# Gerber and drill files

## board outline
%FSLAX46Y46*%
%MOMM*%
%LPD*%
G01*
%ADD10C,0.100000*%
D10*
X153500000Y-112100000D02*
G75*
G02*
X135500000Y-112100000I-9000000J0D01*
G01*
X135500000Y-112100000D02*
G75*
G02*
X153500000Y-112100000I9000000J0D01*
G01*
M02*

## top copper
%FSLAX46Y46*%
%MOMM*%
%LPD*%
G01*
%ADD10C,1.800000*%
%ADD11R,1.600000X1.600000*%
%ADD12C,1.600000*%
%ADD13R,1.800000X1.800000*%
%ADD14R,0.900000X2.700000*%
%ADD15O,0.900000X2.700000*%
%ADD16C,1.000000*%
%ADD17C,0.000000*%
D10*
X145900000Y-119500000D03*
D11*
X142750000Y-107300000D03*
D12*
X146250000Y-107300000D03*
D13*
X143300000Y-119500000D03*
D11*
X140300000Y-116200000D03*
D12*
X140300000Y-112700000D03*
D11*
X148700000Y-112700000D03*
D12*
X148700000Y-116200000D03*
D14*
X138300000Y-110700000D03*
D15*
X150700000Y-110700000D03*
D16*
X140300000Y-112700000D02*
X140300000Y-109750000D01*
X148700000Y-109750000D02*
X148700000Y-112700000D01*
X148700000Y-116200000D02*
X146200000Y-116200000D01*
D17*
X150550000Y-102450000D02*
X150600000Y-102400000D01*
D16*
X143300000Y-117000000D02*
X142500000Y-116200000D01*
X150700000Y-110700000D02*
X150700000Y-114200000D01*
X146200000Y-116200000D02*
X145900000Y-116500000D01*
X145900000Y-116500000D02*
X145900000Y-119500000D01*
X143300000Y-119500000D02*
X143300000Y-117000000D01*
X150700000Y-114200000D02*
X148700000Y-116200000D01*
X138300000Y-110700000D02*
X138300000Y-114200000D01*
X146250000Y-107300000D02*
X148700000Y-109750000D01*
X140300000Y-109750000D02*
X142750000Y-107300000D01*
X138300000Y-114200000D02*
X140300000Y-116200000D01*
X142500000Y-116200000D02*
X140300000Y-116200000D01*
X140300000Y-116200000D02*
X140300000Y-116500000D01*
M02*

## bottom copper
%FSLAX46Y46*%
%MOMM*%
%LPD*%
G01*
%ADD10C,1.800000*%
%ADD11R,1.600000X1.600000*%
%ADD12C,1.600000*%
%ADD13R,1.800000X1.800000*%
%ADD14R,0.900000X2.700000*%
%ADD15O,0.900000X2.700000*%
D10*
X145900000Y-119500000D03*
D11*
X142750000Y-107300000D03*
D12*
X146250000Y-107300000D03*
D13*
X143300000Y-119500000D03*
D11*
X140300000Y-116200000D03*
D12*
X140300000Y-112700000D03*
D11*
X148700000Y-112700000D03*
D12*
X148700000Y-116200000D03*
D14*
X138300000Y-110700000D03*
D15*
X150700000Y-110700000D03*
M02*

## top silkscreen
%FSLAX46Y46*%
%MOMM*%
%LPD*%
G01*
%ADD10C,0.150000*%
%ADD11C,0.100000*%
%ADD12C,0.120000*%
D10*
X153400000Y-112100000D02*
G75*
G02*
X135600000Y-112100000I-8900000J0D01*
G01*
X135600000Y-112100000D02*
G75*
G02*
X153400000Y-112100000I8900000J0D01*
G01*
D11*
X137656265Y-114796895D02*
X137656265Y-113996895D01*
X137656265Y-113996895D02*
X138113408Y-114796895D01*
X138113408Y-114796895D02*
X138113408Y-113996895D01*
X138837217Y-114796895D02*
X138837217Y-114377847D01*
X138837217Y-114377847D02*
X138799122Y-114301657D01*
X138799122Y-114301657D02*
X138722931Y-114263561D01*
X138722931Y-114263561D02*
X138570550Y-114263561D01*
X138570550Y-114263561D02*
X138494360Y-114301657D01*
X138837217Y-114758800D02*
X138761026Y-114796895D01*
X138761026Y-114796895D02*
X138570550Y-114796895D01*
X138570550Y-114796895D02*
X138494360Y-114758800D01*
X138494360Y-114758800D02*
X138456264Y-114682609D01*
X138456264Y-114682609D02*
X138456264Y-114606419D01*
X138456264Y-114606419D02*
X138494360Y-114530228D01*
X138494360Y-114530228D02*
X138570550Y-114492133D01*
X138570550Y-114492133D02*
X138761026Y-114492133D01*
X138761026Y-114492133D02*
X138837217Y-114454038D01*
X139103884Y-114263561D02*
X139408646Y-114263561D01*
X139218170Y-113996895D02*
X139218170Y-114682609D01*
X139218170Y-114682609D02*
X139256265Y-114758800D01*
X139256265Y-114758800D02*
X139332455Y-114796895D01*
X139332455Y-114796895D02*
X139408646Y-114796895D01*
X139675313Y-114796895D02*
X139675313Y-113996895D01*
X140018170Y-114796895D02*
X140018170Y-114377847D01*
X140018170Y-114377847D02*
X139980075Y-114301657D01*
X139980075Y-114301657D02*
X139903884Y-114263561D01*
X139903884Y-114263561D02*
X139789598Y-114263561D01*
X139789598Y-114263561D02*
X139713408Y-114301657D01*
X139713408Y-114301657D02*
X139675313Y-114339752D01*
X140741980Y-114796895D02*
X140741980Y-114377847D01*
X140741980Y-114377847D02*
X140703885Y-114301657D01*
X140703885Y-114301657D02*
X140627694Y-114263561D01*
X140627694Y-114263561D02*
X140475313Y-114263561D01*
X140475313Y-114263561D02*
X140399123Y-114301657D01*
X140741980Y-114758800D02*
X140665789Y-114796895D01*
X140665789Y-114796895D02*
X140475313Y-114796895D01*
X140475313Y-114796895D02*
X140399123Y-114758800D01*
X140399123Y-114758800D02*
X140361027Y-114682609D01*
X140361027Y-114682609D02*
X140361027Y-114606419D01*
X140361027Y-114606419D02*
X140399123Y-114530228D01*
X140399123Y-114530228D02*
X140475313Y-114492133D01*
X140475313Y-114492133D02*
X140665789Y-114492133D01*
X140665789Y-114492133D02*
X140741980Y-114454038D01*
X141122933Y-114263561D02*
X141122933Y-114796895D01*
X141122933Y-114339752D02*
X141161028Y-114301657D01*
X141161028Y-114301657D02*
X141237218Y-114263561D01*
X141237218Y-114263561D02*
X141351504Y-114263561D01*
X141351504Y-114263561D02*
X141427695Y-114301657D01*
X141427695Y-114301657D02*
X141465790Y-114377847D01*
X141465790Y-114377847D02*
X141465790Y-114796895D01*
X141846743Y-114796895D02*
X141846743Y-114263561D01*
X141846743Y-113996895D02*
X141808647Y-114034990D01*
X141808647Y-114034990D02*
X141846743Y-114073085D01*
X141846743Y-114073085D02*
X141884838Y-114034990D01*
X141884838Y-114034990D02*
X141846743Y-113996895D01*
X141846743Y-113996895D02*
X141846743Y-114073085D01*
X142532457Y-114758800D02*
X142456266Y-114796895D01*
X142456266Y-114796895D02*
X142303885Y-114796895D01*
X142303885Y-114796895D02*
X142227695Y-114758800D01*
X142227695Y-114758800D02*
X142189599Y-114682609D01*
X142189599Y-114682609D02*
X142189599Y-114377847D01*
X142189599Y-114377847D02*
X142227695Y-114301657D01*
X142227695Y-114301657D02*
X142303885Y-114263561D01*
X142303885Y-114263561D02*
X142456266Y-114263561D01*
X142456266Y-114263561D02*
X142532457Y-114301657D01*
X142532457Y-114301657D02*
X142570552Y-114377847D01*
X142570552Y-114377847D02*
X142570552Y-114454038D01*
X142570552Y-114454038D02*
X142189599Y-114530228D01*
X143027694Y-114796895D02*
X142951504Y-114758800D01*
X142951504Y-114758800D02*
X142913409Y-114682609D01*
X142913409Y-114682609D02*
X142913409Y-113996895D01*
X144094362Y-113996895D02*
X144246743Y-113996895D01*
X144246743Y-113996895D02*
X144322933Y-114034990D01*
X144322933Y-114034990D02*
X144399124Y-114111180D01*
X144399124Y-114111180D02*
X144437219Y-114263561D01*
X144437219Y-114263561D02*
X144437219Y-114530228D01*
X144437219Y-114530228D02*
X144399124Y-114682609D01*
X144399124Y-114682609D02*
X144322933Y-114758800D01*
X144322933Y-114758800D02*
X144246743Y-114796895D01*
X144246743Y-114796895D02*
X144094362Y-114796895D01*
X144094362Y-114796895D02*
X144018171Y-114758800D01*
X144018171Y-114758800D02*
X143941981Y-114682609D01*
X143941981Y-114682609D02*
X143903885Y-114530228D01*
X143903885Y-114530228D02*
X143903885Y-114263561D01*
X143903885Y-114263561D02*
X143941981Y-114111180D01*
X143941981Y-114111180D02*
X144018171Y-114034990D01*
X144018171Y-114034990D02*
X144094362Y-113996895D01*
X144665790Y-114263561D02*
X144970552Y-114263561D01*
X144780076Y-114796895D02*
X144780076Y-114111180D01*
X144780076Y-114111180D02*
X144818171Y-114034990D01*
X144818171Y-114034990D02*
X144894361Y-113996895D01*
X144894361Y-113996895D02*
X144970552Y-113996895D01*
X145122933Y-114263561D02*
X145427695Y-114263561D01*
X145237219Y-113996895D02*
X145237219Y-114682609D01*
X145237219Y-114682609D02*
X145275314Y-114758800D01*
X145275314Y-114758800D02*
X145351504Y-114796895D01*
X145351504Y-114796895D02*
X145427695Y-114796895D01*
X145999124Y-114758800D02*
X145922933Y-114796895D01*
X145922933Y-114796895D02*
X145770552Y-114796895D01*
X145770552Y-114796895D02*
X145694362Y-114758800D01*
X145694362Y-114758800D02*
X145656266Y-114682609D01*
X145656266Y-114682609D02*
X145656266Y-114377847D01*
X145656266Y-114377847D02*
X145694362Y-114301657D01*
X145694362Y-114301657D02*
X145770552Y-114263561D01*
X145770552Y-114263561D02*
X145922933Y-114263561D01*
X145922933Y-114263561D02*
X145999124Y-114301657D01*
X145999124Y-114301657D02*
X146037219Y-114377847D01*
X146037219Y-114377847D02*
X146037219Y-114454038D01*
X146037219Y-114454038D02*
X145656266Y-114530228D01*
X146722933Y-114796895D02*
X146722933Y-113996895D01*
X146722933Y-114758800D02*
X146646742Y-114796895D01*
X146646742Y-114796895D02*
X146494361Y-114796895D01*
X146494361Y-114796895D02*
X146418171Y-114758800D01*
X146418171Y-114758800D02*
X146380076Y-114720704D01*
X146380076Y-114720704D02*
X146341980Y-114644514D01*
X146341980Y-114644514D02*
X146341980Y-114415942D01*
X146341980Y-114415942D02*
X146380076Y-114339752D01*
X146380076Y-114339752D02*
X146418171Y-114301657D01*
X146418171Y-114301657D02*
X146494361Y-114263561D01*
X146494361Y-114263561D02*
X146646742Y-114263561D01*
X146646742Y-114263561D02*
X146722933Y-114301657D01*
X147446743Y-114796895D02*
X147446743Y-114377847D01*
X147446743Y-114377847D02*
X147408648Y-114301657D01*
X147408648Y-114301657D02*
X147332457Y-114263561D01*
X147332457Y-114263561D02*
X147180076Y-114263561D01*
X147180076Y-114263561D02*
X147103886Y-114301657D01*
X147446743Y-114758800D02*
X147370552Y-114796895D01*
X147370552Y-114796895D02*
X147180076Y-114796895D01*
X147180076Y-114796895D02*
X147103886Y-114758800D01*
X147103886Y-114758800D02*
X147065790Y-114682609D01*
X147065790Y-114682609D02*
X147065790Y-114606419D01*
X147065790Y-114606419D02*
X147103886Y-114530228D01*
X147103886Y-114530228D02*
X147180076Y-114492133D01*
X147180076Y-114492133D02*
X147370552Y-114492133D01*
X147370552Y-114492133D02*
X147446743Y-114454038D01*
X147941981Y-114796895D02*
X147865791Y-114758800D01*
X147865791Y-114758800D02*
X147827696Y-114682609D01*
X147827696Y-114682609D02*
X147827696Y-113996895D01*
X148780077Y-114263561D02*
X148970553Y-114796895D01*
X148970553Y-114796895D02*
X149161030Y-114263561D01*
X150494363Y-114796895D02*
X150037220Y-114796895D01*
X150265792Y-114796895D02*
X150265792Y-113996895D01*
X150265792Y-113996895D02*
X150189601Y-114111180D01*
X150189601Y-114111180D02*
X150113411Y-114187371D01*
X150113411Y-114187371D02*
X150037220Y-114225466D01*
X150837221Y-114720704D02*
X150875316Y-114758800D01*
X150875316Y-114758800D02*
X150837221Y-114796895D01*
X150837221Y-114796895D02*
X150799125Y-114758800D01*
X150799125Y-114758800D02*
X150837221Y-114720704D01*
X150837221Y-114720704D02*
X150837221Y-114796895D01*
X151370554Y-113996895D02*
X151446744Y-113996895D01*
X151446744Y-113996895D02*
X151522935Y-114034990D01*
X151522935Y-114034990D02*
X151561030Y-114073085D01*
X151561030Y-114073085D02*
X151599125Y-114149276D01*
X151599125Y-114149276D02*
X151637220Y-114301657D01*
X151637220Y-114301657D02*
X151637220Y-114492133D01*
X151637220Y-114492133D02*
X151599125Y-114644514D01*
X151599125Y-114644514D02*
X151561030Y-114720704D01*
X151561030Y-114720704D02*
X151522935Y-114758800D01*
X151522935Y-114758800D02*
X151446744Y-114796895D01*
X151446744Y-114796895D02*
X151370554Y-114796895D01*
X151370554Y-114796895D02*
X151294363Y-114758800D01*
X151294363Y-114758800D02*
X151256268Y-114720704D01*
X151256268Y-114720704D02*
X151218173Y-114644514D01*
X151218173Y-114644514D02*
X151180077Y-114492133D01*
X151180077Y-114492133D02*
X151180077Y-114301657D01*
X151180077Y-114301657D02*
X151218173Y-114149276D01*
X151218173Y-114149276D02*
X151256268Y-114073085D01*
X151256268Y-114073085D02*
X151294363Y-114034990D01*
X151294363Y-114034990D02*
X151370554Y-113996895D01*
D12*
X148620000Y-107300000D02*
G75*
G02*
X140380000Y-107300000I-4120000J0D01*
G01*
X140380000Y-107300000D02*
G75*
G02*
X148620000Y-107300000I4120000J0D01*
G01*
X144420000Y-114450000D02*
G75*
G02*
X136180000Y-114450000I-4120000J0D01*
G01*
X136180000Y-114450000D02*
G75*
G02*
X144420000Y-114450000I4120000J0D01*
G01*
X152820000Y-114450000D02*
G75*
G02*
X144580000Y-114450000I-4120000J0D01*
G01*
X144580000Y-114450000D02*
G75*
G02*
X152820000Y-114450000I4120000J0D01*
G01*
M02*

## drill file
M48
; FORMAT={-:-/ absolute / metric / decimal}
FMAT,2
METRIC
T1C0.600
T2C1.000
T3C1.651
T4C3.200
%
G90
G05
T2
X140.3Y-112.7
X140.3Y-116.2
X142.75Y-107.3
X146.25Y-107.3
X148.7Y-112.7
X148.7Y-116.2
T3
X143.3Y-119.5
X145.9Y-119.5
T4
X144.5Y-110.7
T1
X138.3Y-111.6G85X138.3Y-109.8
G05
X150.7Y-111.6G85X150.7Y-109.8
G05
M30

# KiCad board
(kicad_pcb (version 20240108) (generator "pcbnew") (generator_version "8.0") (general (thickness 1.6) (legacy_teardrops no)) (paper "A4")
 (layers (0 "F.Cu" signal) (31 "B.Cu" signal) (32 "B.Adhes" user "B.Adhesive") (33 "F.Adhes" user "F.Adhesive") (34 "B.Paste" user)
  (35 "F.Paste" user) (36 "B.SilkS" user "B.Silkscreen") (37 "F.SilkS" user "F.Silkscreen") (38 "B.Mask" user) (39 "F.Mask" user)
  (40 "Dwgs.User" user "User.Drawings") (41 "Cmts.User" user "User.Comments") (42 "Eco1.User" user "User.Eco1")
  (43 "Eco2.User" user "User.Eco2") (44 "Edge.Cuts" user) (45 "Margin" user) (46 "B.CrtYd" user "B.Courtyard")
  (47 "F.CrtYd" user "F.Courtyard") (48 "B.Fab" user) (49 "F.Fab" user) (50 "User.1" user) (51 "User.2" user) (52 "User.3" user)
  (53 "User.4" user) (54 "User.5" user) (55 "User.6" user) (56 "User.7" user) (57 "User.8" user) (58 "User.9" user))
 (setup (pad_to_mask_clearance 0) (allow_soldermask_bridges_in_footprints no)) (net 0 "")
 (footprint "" (layer "F.Cu") (at 145.9 119.5)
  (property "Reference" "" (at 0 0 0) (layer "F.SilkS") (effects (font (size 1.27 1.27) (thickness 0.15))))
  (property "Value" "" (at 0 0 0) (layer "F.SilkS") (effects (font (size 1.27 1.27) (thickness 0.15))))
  (pad "2" thru_hole circle (at 0 0) (size 1.8 1.8) (drill 1.651) (layers "*.Cu" "*.Mask") (remove_unused_layers no)))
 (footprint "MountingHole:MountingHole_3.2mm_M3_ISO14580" (layer "F.Cu") (at 144.5 110.7)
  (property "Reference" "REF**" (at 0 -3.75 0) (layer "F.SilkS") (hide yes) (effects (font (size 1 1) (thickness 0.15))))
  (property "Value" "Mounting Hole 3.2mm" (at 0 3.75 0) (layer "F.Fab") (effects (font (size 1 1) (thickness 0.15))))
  (pad "" np_thru_hole circle (at 0 0) (size 3.2 3.2) (drill 3.2) (layers "F&B.Cu" "*.Mask" "B.Paste")))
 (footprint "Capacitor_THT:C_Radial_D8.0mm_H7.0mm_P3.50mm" (layer "F.Cu") (at 142.75 107.3)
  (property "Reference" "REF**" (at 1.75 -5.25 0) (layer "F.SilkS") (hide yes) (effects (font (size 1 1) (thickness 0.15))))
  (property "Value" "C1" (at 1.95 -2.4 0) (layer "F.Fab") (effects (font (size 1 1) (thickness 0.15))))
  (fp_circle (center 1.75 0) (end 5.87 0) (stroke (width 0.12) (type solid)) (fill none) (layer "F.SilkS"))
  (pad "1" thru_hole rect (at 0 0) (size 1.6 1.6) (drill 1) (layers "*.Cu" "*.Mask") (remove_unused_layers no))
  (pad "2" thru_hole circle (at 3.5 0) (size 1.6 1.6) (drill 1) (layers "*.Cu" "*.Mask") (remove_unused_layers no)))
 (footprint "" (layer "F.Cu") (at 143.3 119.5)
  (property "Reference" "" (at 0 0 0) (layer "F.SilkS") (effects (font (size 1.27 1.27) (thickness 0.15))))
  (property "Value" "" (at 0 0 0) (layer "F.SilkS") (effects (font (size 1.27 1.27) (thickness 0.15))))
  (pad "1" thru_hole rect (at 0 0) (size 1.8 1.8) (drill 1.651) (layers "*.Cu" "*.Mask") (remove_unused_layers no)))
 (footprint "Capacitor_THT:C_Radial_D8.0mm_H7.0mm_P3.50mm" (layer "F.Cu") (at 140.3 116.2 90)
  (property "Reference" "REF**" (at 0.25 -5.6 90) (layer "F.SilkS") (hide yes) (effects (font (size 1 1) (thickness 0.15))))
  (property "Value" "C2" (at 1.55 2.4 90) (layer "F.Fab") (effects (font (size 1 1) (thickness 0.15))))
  (fp_circle (center 1.75 0) (end 5.87 0) (stroke (width 0.12) (type solid)) (fill none) (layer "F.SilkS"))
  (pad "1" thru_hole rect (at 0 0 90) (size 1.6 1.6) (drill 1) (layers "*.Cu" "*.Mask") (remove_unused_layers no))
  (pad "2" thru_hole circle (at 3.5 0 90) (size 1.6 1.6) (drill 1) (layers "*.Cu" "*.Mask") (remove_unused_layers no)))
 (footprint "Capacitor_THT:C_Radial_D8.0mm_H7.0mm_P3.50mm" (layer "F.Cu") (at 148.7 112.7 -90)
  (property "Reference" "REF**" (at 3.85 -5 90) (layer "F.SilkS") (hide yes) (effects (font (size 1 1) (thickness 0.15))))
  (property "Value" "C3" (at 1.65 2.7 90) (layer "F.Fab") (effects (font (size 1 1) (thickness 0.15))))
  (fp_circle (center 1.75 0) (end 5.87 0) (stroke (width 0.12) (type solid)) (fill none) (layer "F.SilkS"))
  (pad "1" thru_hole rect (at 0 0 270) (size 1.6 1.6) (drill 1) (layers "*.Cu" "*.Mask") (remove_unused_layers no))
  (pad "2" thru_hole circle (at 3.5 0 270) (size 1.6 1.6) (drill 1) (layers "*.Cu" "*.Mask") (remove_unused_layers no)))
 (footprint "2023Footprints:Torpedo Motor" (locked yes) (layer "B.Cu") (at 144.5 110.7 90)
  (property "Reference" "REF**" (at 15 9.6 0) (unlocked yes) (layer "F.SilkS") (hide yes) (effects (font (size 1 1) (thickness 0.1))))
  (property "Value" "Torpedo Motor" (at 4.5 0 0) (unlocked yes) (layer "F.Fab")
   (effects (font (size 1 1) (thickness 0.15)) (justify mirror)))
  (pad "1" thru_hole rect (at 0 -6.2 90) (size 2.7 0.9) (drill oval 2.4 0.6) (layers "*.Cu" "*.Mask") (remove_unused_layers no))
  (pad "2" thru_hole oval (at 0 6.2 90) (size 2.7 0.9) (drill oval 2.4 0.6) (layers "*.Cu" "*.Mask") (remove_unused_layers no)))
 (gr_circle (center 144.5 112.1) (end 153.4 112.1) (stroke (width 0.15) (type default)) (fill none) (layer "F.SilkS"))
 (gr_circle (center 144.5 112.1) (end 153.5 112.1) (stroke (width 0.1) (type default)) (fill none) (layer "Edge.Cuts"))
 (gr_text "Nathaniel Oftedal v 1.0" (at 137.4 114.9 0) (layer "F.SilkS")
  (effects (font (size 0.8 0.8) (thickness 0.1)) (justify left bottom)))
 (segment (start 140.3 112.7) (end 140.3 109.75) (width 1) (layer "F.Cu") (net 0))
 (segment (start 148.7 109.75) (end 148.7 112.7) (width 1) (layer "F.Cu") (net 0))
 (segment (start 148.7 116.2) (end 146.2 116.2) (width 1) (layer "F.Cu") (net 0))
 (segment (start 150.55 102.45) (end 150.6 102.4) (width 0) (layer "F.Cu") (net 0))
 (segment (start 143.3 117) (end 142.5 116.2) (width 1) (layer "F.Cu") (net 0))
 (segment (start 150.7 110.7) (end 150.7 114.2) (width 1) (layer "F.Cu") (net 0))
 (segment (start 146.2 116.2) (end 145.9 116.5) (width 1) (layer "F.Cu") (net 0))
 (segment (start 145.9 116.5) (end 145.9 119.5) (width 1) (layer "F.Cu") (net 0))
 (segment (start 143.3 119.5) (end 143.3 117) (width 1) (layer "F.Cu") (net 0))
 (segment (start 150.7 114.2) (end 148.7 116.2) (width 1) (layer "F.Cu") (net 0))
 (segment (start 138.3 110.7) (end 138.3 114.2) (width 1) (layer "F.Cu") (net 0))
 (segment (start 146.25 107.3) (end 148.7 109.75) (width 1) (layer "F.Cu") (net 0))
 (segment (start 140.3 109.75) (end 142.75 107.3) (width 1) (layer "F.Cu") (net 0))
 (segment (start 138.3 114.2) (end 140.3 116.2) (width 1) (layer "F.Cu") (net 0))
 (segment (start 142.5 116.2) (end 140.3 116.2) (width 1) (layer "F.Cu") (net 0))
 (segment (start 140.3 116.2) (end 140.3 116.5) (width 1) (layer "F.Cu") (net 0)))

